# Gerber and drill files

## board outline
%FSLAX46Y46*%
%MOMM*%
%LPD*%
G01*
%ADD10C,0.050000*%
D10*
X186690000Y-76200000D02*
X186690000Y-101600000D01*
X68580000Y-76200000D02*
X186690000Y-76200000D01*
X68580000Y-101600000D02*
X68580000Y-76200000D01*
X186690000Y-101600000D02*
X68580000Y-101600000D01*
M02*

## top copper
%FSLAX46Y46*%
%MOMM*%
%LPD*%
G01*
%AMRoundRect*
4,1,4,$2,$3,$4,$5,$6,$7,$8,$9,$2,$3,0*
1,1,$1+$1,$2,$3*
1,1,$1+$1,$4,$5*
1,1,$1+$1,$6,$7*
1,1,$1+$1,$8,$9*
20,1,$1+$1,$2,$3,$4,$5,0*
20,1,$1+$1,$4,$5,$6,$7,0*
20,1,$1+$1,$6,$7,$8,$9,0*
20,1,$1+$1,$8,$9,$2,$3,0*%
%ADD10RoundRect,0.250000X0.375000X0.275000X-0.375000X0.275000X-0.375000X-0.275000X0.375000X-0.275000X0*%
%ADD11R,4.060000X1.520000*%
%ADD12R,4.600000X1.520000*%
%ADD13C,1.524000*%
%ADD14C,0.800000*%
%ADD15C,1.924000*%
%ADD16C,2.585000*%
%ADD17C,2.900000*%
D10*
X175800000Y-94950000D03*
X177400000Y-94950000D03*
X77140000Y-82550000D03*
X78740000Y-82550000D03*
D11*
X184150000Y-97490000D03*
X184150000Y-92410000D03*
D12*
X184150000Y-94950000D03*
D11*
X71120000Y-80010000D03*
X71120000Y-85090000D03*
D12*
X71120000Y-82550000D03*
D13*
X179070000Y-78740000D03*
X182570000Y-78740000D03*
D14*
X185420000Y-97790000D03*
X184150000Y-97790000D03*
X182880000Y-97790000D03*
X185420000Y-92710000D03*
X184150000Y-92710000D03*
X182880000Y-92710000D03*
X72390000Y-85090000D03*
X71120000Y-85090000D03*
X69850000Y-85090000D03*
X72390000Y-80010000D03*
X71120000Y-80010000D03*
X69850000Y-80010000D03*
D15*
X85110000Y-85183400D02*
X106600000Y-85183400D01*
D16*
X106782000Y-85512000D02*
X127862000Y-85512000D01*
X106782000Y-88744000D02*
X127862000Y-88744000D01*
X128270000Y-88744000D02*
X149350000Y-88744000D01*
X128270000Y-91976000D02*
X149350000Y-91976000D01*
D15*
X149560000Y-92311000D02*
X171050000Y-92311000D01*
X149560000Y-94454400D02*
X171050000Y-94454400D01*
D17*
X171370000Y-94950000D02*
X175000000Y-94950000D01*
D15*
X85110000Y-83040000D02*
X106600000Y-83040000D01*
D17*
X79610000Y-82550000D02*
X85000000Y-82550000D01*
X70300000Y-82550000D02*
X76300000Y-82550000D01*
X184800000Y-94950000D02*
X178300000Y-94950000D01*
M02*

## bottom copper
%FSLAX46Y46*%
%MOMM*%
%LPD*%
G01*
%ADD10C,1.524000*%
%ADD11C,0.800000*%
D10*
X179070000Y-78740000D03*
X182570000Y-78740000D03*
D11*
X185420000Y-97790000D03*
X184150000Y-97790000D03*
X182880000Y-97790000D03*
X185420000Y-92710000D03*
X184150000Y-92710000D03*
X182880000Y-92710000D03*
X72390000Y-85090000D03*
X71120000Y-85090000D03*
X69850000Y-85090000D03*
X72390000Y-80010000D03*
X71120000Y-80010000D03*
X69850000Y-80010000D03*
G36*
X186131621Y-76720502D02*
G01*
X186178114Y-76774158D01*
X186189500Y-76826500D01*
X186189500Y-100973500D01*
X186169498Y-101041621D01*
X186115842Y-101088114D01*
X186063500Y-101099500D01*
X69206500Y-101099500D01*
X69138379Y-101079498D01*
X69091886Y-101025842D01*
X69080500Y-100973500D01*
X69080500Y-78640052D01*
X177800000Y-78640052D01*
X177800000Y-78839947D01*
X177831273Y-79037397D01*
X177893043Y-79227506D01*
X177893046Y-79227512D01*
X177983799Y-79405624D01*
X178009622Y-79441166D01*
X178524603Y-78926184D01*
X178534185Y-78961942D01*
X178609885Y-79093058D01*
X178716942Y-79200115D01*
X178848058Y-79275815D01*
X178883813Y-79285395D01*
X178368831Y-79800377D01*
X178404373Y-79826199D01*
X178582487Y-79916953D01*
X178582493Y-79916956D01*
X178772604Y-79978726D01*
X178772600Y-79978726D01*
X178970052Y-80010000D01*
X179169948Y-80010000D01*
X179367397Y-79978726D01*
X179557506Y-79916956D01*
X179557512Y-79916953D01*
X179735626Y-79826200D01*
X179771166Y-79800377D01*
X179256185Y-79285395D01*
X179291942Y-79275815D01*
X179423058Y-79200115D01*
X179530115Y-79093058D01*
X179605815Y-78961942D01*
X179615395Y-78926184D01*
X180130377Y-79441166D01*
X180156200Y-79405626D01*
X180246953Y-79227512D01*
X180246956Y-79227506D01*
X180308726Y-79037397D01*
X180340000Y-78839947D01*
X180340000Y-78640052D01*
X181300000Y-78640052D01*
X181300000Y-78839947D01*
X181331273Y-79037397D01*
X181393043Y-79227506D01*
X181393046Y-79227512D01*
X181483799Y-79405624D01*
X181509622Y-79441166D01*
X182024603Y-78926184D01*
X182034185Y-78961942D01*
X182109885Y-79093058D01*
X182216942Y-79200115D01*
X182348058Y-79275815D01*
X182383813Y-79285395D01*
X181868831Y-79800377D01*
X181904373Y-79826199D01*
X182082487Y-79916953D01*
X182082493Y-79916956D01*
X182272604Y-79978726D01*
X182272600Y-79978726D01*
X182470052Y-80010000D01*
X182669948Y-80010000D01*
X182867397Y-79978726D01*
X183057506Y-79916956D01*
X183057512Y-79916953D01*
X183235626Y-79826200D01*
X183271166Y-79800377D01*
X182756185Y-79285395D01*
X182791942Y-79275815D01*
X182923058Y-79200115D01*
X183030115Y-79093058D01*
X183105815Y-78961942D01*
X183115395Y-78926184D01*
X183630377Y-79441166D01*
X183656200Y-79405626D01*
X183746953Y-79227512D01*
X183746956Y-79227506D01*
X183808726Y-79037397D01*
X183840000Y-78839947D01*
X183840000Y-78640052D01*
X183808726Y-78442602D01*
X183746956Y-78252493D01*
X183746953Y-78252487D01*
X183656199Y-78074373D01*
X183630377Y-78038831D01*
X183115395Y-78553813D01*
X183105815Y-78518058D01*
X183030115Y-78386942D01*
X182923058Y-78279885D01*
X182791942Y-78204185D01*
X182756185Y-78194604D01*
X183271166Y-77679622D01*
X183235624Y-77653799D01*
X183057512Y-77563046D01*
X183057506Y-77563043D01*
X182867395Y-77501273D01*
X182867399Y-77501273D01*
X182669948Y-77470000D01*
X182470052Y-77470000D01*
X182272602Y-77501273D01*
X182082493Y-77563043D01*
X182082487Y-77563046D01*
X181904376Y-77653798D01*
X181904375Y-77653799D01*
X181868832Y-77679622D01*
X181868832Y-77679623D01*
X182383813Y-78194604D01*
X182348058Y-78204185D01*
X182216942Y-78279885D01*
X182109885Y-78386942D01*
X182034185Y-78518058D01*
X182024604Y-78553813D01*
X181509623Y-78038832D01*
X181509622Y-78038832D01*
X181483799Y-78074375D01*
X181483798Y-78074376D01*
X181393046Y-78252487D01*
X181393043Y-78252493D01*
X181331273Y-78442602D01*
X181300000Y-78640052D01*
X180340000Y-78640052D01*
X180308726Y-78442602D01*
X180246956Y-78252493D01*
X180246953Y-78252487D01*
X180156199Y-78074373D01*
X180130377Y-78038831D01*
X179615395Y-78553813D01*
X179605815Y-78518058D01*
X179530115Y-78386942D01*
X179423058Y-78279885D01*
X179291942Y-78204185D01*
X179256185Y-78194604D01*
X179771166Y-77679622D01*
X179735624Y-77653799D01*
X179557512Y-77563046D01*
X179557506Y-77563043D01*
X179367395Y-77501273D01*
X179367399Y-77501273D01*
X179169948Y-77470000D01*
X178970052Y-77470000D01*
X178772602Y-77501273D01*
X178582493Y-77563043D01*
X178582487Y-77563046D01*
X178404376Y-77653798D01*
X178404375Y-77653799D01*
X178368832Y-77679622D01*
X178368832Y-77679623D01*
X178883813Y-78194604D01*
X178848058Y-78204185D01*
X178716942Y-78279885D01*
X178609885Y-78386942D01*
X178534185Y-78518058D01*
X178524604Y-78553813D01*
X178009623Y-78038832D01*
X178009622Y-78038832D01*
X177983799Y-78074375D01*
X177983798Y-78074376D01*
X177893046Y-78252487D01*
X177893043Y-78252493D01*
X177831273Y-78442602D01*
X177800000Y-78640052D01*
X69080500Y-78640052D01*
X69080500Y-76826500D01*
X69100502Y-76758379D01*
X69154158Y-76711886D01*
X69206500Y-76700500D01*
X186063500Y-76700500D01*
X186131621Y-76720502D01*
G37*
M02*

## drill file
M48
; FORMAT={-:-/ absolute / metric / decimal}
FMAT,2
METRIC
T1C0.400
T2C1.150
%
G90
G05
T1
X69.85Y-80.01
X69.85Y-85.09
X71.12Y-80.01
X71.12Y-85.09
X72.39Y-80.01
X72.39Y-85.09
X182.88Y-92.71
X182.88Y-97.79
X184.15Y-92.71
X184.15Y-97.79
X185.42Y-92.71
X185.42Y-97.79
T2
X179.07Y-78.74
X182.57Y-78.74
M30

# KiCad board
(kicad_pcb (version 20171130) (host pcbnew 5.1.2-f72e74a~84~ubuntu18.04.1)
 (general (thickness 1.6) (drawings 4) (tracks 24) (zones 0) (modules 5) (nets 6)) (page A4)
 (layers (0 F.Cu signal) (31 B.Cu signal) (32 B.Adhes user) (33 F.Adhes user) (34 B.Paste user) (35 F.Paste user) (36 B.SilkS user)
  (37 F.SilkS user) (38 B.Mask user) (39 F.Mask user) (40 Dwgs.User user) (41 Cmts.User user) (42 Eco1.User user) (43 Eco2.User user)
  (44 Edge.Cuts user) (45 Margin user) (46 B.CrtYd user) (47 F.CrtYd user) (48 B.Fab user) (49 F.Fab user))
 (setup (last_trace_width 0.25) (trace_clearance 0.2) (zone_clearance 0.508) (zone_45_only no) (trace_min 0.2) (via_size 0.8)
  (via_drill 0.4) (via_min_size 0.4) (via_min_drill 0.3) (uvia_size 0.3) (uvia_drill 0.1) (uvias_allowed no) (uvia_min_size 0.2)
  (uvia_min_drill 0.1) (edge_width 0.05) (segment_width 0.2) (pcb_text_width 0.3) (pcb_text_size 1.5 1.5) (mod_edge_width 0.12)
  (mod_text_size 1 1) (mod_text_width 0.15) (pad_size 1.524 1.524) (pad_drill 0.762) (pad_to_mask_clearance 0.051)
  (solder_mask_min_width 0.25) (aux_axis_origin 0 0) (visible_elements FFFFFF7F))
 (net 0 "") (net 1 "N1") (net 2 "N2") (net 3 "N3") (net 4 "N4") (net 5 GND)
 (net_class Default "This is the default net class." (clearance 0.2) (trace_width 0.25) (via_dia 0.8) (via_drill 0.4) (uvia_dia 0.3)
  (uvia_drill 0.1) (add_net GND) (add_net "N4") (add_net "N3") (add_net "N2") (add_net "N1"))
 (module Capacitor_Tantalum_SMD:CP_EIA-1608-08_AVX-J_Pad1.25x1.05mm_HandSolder (layer F.Cu) (at 176.6 94.95 180)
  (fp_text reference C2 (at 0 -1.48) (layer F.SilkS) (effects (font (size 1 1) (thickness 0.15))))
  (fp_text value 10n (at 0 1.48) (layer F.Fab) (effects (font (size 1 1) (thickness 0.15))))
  (pad 2 smd roundrect (at 0.8 0 180) (size 1.25 1.05) (layers F.Cu F.Paste F.Mask) (roundrect_rratio 0.238095) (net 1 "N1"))
  (pad 1 smd roundrect (at -0.8 0 180) (size 1.25 1.05) (layers F.Cu F.Paste F.Mask) (roundrect_rratio 0.238095) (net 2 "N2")))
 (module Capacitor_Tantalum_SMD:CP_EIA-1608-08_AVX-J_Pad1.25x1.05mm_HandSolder (layer F.Cu) (at 77.94 82.55 180)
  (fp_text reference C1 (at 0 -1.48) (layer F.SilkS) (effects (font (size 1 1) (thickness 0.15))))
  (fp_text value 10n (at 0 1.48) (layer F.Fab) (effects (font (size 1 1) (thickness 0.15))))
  (pad 2 smd roundrect (at 0.8 0 180) (size 1.25 1.05) (layers F.Cu F.Paste F.Mask) (roundrect_rratio 0.238095) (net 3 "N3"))
  (pad 1 smd roundrect (at -0.8 0 180) (size 1.25 1.05) (layers F.Cu F.Paste F.Mask) (roundrect_rratio 0.238095) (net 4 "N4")))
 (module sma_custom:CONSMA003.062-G (layer F.Cu) (at 187.96 97.49)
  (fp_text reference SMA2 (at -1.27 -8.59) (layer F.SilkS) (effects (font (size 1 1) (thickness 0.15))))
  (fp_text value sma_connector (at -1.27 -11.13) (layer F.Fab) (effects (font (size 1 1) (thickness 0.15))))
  (pad 3 smd rect (at -3.81 0) (size 4.06 1.52) (layers F.Cu F.Paste F.Mask) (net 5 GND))
  (pad 2 smd rect (at -3.81 -5.08) (size 4.06 1.52) (layers F.Cu F.Paste F.Mask) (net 5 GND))
  (pad 1 smd rect (at -3.81 -2.54) (size 4.6 1.52) (layers F.Cu F.Paste F.Mask) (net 2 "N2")))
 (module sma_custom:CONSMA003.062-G (layer F.Cu) (at 67.31 80.01 180)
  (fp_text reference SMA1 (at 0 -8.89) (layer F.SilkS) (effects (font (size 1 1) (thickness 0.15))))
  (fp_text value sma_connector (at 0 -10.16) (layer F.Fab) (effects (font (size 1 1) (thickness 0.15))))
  (pad 3 smd rect (at -3.81 0 180) (size 4.06 1.52) (layers F.Cu F.Paste F.Mask) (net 5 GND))
  (pad 2 smd rect (at -3.81 -5.08 180) (size 4.06 1.52) (layers F.Cu F.Paste F.Mask) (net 5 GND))
  (pad 1 smd rect (at -3.81 -2.54 180) (size 4.6 1.52) (layers F.Cu F.Paste F.Mask) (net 3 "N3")))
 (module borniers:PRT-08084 (layer F.Cu) (at 179.07 73.66 180)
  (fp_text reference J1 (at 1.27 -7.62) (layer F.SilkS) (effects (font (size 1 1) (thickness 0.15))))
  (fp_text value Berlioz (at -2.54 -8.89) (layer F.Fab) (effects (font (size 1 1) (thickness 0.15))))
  (pad 2 thru_hole circle (at 0 -5.08 180) (size 1.524 1.524) (drill 1.15) (layers *.Cu *.Mask) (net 5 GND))
  (pad 1 thru_hole circle (at -3.5 -5.08 180) (size 1.524 1.524) (drill 1.15) (layers *.Cu *.Mask) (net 5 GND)))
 (gr_line (start 186.69 76.2) (end 186.69 101.6) (layer Edge.Cuts) (width 0.05))
 (gr_line (start 68.58 76.2) (end 186.69 76.2) (layer Edge.Cuts) (width 0.05))
 (gr_line (start 68.58 101.6) (end 68.58 76.2) (layer Edge.Cuts) (width 0.05))
 (gr_line (start 186.69 101.6) (end 68.58 101.6) (layer Edge.Cuts) (width 0.05))
 (segment (start 85.11 85.1834) (end 106.6 85.1834) (width 1.924) (layer F.Cu) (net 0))
 (segment (start 106.782 85.512) (end 127.862 85.512) (width 2.585) (layer F.Cu) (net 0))
 (segment (start 106.782 88.744) (end 127.862 88.744) (width 2.585) (layer F.Cu) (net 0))
 (segment (start 128.27 88.744) (end 149.35 88.744) (width 2.585) (layer F.Cu) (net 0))
 (segment (start 128.27 91.976) (end 149.35 91.976) (width 2.585) (layer F.Cu) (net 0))
 (segment (start 149.56 92.311) (end 171.05 92.311) (width 1.924) (layer F.Cu) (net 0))
 (via (at 185.42 97.79) (size 0.8) (drill 0.4) (layers F.Cu B.Cu) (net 5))
 (via (at 184.15 97.79) (size 0.8) (drill 0.4) (layers F.Cu B.Cu) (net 5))
 (via (at 182.88 97.79) (size 0.8) (drill 0.4) (layers F.Cu B.Cu) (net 5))
 (via (at 185.42 92.71) (size 0.8) (drill 0.4) (layers F.Cu B.Cu) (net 5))
 (via (at 184.15 92.71) (size 0.8) (drill 0.4) (layers F.Cu B.Cu) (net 5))
 (via (at 182.88 92.71) (size 0.8) (drill 0.4) (layers F.Cu B.Cu) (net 5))
 (via (at 72.39 85.09) (size 0.8) (drill 0.4) (layers F.Cu B.Cu) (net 5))
 (via (at 71.12 85.09) (size 0.8) (drill 0.4) (layers F.Cu B.Cu) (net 5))
 (via (at 69.85 85.09) (size 0.8) (drill 0.4) (layers F.Cu B.Cu) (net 5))
 (via (at 72.39 80.01) (size 0.8) (drill 0.4) (layers F.Cu B.Cu) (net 5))
 (via (at 71.12 80.01) (size 0.8) (drill 0.4) (layers F.Cu B.Cu) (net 5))
 (via (at 69.85 80.01) (size 0.8) (drill 0.4) (layers F.Cu B.Cu) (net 5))
 (segment (start 149.56 94.4544) (end 171.05 94.4544) (width 1.924) (layer F.Cu) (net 1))
 (segment (start 171.37 94.95) (end 175 94.95) (width 2.9) (layer F.Cu) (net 1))
 (segment (start 85.11 83.04) (end 106.6 83.04) (width 1.924) (layer F.Cu) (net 4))
 (segment (start 79.61 82.55) (end 85 82.55) (width 2.9) (layer F.Cu) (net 4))
 (segment (start 70.3 82.55) (end 76.3 82.55) (width 2.9) (layer F.Cu) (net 3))
 (segment (start 184.8 94.95) (end 178.3 94.95) (width 2.9) (layer F.Cu) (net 2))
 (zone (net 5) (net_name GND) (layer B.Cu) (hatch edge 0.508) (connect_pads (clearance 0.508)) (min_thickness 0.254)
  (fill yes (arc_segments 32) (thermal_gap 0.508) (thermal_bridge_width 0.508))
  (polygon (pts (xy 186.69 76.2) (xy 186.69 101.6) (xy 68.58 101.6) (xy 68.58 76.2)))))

